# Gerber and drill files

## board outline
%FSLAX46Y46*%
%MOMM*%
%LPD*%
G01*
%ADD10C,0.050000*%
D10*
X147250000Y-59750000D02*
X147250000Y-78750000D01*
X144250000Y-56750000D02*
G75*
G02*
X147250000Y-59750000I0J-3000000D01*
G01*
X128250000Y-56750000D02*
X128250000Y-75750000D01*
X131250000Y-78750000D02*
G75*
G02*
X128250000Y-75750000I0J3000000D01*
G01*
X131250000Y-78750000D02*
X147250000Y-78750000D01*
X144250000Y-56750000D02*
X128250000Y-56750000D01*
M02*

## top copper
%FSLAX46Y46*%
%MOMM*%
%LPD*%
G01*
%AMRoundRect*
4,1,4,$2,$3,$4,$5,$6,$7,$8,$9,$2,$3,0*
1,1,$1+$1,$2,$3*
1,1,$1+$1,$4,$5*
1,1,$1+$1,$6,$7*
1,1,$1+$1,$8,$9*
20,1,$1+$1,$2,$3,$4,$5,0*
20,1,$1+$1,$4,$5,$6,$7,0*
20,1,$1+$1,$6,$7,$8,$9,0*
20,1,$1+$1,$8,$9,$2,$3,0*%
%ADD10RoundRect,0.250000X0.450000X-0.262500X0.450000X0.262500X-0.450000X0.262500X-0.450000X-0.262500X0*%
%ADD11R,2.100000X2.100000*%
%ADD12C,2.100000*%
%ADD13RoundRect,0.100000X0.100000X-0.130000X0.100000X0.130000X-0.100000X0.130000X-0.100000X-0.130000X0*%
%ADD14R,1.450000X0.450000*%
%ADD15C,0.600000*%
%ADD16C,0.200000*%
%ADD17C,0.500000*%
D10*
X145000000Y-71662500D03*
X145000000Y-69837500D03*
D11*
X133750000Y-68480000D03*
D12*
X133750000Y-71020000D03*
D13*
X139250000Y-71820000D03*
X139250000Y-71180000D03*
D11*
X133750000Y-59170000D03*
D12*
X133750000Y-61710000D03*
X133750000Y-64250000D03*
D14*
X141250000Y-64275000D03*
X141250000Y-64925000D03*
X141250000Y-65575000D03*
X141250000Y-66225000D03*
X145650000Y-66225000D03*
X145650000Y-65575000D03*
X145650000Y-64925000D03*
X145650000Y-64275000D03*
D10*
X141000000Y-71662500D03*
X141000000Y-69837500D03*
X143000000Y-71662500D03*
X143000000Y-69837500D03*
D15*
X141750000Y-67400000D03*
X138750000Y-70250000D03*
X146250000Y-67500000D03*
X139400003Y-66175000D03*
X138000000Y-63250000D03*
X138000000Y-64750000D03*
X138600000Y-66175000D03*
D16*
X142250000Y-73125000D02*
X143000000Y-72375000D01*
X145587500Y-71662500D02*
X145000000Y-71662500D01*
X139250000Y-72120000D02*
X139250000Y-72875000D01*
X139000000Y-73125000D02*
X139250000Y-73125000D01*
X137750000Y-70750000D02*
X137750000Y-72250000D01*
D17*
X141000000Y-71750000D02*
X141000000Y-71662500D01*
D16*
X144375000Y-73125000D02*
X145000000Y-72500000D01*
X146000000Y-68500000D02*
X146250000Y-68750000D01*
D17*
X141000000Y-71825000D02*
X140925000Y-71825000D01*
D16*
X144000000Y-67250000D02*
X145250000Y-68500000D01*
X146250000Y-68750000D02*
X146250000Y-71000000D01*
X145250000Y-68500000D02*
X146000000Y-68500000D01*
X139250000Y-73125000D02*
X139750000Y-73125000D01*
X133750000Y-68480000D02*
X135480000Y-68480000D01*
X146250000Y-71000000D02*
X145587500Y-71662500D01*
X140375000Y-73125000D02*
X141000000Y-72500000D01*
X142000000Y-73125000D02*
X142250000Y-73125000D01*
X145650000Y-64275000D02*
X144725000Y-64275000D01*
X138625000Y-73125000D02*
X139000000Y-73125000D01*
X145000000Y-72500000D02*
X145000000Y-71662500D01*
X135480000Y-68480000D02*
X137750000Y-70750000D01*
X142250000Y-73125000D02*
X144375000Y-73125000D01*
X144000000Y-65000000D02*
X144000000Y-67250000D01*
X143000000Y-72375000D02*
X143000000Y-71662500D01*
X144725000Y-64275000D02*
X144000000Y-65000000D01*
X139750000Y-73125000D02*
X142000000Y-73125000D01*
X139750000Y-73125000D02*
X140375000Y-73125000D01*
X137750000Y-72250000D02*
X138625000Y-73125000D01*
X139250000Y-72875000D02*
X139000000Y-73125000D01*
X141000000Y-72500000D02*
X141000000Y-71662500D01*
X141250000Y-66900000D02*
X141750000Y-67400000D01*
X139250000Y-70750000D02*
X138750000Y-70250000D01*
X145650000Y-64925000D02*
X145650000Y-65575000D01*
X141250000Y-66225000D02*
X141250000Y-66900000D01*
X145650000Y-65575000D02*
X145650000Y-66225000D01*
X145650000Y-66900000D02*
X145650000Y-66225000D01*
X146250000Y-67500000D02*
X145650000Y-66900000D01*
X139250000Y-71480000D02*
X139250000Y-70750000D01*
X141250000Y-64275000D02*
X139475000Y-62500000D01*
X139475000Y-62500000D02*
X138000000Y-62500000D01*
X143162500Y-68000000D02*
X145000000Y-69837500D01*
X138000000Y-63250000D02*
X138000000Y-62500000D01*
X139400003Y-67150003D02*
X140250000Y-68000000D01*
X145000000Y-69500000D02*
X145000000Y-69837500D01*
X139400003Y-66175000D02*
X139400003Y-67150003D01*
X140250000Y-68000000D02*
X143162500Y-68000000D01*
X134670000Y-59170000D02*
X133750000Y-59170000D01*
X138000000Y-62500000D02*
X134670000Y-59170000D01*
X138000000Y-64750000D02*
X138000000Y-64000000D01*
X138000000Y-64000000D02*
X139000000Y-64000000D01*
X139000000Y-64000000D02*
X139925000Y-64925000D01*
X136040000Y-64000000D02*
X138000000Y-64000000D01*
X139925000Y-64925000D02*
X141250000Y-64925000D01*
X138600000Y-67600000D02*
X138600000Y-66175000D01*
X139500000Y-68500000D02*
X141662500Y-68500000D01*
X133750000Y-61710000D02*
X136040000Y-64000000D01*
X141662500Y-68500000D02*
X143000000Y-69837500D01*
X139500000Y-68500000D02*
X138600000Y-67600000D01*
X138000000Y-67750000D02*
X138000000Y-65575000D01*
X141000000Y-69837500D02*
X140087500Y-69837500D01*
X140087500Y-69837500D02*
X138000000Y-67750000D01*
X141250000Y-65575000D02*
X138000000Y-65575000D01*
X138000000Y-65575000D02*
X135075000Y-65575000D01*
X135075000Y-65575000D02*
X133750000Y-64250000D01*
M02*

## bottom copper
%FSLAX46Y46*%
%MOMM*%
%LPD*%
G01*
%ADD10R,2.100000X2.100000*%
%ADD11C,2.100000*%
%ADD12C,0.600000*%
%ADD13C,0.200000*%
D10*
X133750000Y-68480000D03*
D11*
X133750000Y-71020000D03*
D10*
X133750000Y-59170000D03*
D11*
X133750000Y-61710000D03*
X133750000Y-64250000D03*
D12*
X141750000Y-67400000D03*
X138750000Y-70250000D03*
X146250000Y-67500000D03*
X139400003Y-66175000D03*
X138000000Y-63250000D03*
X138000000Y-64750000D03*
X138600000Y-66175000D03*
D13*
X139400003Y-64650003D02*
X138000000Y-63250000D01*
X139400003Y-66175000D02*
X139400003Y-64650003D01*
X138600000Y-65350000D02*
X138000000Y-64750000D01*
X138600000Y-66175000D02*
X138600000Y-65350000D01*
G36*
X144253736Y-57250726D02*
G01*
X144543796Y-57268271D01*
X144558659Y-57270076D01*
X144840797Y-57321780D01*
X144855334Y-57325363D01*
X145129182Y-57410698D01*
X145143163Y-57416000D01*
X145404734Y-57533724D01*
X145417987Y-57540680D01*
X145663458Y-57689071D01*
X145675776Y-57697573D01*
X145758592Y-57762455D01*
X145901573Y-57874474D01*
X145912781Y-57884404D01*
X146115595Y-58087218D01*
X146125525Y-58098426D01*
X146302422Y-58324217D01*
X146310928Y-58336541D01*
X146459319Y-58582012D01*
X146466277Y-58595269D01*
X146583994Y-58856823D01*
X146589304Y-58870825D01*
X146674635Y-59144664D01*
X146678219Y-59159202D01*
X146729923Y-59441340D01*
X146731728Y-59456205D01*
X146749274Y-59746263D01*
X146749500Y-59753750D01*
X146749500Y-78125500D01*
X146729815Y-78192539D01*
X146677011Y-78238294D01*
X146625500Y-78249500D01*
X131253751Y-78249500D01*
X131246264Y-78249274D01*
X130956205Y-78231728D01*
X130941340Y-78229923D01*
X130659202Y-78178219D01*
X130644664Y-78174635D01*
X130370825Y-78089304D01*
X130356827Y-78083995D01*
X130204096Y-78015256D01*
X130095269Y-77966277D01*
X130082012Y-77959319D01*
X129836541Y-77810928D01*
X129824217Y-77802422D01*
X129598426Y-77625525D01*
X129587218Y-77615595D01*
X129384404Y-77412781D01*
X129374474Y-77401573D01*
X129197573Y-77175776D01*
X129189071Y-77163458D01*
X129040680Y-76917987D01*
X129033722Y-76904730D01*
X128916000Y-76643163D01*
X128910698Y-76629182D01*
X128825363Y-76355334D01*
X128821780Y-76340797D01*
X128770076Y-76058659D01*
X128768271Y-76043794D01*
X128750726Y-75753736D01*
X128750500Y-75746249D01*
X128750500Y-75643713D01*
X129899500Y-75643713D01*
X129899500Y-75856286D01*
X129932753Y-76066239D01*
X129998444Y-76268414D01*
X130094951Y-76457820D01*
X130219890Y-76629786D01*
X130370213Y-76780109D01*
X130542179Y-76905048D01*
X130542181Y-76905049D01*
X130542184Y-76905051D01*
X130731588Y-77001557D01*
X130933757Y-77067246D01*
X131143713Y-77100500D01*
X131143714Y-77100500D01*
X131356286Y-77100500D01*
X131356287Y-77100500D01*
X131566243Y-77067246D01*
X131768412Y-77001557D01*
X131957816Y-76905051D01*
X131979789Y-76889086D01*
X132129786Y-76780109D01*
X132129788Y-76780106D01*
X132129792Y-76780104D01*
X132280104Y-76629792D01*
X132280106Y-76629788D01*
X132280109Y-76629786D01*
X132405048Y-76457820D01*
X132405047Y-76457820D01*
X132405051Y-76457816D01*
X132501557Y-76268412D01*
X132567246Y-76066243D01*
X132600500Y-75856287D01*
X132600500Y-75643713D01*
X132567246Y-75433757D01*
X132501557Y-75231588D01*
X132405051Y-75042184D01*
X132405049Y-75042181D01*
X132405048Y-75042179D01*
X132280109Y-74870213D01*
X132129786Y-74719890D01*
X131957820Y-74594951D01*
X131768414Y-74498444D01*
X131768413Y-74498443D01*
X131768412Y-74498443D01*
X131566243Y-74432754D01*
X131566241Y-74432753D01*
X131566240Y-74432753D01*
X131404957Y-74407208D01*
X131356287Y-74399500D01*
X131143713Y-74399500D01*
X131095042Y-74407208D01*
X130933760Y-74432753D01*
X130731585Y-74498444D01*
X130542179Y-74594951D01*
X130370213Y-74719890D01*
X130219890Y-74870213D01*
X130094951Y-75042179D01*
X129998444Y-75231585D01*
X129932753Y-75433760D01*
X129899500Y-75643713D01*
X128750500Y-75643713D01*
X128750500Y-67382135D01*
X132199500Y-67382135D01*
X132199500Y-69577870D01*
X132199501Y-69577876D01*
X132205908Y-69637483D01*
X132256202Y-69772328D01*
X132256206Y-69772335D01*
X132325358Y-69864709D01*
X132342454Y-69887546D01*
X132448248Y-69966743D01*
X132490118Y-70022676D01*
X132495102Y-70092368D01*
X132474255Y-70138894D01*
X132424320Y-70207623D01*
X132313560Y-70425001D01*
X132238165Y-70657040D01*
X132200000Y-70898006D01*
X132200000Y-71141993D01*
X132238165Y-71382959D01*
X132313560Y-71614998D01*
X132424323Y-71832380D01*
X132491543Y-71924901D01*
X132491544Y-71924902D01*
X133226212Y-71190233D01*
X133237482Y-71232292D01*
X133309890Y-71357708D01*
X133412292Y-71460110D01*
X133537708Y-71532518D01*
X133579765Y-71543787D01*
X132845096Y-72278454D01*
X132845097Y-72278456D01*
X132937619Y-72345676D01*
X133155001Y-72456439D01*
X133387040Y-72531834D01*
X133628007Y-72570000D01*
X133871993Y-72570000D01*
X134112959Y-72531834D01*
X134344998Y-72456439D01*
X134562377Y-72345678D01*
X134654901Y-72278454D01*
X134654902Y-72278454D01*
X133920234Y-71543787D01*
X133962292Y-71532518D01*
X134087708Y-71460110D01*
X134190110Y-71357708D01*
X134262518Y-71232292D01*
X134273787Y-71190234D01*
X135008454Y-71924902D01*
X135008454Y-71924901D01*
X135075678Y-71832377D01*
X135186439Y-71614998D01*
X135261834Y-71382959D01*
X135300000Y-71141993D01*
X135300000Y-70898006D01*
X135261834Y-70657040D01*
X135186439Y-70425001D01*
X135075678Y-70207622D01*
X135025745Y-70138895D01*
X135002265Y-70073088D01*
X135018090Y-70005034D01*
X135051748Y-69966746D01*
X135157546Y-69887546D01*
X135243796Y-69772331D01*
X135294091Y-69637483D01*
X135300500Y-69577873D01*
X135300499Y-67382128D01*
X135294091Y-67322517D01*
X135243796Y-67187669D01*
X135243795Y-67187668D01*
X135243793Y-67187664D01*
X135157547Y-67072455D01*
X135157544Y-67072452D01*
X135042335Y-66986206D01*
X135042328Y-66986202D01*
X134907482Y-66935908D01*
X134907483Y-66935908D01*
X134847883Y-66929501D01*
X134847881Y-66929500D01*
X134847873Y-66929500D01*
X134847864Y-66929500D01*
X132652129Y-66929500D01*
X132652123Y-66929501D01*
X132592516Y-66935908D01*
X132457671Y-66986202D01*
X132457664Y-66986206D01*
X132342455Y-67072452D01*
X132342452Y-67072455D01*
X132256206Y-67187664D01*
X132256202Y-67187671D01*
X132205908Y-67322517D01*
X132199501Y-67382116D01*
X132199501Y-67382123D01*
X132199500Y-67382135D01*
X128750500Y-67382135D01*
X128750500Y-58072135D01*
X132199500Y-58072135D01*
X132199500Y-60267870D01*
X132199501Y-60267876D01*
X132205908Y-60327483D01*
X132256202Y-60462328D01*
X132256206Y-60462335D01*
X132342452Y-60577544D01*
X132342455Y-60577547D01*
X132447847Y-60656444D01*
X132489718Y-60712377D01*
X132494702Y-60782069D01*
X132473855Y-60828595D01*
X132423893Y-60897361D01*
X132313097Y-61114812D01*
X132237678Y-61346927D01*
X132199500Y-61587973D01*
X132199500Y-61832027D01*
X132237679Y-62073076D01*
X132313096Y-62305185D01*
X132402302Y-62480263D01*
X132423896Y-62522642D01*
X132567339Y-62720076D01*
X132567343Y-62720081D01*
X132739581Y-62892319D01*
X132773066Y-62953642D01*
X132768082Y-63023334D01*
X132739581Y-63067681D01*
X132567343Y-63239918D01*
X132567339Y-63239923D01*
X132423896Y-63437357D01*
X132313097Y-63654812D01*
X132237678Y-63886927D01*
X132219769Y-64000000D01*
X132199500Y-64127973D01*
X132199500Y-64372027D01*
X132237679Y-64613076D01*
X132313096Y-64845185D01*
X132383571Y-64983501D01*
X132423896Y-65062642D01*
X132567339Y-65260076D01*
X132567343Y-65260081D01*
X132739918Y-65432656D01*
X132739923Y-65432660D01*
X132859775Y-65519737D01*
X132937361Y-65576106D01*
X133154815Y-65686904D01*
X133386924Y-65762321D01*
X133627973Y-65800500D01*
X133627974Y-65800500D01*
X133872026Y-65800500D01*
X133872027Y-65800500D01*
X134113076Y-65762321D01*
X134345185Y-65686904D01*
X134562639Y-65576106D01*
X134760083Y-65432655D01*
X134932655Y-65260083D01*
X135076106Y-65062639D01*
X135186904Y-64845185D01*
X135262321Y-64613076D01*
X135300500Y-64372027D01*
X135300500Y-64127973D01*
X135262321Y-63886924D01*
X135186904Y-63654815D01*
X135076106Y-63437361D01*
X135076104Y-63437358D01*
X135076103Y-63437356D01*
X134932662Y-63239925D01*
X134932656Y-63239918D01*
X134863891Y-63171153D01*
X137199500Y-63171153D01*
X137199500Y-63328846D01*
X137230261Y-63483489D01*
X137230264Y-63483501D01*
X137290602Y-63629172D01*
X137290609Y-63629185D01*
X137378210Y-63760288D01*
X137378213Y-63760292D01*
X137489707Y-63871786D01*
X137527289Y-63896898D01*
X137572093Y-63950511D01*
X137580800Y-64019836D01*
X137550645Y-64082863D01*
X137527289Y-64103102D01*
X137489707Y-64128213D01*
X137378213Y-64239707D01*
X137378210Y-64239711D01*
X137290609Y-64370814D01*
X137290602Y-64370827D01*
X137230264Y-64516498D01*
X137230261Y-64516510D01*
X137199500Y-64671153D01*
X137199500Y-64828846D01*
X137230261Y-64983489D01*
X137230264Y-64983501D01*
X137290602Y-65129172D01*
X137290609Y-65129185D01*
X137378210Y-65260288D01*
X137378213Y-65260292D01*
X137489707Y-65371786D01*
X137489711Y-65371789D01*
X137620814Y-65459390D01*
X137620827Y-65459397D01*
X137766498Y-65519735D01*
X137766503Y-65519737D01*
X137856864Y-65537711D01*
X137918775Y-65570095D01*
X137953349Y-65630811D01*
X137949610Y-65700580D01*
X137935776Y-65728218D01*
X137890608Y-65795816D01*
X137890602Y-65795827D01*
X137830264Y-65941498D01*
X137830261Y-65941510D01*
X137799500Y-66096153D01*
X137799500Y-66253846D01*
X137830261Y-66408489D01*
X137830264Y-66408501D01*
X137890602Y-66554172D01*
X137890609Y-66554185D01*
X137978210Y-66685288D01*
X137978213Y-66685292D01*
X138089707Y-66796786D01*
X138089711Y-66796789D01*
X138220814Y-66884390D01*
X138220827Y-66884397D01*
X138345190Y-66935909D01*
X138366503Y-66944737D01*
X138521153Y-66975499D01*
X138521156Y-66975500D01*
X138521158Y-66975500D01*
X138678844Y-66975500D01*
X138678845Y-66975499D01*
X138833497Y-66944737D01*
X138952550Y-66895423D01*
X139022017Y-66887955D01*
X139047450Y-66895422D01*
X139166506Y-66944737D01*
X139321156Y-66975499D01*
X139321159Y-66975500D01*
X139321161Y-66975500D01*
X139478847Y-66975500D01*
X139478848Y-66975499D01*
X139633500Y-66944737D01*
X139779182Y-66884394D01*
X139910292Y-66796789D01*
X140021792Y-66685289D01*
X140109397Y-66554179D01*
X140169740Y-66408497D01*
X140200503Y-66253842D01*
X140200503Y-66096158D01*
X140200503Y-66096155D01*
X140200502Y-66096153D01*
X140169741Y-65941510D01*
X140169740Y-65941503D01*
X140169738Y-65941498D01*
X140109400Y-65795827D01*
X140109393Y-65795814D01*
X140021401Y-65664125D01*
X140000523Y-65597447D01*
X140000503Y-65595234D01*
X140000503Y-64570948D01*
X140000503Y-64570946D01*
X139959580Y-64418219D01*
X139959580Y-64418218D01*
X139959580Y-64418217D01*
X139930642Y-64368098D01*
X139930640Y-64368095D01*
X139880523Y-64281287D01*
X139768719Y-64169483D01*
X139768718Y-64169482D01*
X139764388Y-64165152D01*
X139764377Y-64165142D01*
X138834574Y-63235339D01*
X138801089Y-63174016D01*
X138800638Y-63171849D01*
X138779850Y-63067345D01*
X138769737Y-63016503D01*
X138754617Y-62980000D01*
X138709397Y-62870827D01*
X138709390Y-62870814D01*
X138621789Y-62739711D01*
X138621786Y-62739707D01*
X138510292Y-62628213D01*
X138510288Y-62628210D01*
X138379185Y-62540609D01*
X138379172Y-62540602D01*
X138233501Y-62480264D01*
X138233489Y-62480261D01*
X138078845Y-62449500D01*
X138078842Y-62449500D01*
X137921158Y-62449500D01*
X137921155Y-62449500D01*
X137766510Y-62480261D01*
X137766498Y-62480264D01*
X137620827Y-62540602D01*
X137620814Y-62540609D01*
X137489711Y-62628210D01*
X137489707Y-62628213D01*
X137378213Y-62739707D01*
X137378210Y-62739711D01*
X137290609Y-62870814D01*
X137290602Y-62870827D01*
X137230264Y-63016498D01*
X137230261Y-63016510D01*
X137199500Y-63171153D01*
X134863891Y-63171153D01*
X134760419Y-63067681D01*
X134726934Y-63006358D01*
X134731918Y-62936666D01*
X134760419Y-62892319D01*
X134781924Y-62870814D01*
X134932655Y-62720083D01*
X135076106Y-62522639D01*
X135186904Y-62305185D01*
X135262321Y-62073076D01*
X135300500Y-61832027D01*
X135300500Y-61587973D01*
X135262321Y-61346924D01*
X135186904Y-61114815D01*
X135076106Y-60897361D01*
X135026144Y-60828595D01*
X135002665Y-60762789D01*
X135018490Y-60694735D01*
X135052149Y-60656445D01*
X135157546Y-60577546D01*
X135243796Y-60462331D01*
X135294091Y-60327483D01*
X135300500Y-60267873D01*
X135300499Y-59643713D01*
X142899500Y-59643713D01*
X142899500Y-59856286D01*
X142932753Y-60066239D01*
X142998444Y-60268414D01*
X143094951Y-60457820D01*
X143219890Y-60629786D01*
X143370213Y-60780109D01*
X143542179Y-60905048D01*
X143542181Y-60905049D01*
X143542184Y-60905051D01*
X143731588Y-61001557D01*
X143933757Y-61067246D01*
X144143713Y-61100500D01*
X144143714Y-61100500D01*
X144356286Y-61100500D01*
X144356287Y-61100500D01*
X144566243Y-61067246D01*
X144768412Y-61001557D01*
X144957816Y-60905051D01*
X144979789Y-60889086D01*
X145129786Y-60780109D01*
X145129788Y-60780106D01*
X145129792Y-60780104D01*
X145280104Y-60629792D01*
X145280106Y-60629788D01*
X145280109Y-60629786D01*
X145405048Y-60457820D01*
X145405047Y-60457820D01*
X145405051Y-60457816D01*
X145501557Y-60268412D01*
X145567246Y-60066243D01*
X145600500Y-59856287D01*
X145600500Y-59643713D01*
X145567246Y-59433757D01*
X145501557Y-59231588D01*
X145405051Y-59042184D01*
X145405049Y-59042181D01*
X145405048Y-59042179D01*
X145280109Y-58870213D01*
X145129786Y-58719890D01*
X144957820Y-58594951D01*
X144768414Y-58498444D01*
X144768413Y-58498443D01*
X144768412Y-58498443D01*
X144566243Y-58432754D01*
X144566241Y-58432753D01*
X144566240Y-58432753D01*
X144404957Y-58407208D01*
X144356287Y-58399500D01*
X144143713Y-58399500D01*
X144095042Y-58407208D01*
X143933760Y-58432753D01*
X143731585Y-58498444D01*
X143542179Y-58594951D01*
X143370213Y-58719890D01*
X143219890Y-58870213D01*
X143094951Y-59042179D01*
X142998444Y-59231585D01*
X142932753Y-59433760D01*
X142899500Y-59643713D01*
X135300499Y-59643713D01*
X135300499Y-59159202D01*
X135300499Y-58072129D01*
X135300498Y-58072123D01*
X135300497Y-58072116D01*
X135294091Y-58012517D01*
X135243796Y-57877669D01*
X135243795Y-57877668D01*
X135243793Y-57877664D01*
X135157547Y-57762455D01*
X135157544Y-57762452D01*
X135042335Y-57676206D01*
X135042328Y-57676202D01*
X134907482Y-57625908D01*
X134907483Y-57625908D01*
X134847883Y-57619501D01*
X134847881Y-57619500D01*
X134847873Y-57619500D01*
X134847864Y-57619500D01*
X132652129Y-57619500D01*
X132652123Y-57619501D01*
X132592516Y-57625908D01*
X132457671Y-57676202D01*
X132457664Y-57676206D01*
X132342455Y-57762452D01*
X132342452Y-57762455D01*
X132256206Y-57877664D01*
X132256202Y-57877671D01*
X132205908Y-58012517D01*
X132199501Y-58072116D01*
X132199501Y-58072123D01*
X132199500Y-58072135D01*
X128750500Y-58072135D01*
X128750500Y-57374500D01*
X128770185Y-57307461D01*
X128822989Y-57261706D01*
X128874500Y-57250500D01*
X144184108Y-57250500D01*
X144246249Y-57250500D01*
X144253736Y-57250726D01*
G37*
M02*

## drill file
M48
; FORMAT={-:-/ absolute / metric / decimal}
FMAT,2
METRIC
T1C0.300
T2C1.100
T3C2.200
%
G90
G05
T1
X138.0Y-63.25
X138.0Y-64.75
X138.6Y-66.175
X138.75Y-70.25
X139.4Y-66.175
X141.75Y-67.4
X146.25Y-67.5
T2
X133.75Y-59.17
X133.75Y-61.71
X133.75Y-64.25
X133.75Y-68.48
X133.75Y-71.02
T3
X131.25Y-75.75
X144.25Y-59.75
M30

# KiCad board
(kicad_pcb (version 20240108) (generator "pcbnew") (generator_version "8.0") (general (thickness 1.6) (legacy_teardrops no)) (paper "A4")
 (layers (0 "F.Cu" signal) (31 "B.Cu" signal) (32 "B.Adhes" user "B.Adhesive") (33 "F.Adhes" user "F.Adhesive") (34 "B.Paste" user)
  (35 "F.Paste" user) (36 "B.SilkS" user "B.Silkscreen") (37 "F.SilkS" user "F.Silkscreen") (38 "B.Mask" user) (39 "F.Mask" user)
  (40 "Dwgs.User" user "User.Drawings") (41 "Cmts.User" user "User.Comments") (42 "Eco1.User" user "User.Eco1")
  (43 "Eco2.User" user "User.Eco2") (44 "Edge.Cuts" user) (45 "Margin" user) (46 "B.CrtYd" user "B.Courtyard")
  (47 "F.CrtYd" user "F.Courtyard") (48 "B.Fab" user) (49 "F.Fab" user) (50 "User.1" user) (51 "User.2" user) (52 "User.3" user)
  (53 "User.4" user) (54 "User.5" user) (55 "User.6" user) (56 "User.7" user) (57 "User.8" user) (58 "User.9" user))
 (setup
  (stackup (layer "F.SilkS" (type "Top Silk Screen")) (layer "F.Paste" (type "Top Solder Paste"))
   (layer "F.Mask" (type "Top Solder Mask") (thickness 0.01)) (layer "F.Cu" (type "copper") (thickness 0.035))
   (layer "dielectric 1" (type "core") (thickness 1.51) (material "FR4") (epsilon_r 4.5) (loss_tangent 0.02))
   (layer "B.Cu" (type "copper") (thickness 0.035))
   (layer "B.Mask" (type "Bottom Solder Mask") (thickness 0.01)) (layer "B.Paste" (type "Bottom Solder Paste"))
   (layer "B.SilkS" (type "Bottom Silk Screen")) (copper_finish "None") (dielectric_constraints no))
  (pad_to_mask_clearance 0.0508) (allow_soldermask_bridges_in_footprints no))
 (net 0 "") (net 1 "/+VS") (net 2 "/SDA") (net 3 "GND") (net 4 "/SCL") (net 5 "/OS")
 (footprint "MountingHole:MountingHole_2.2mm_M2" (layer "F.Cu") (at 144.25 59.75)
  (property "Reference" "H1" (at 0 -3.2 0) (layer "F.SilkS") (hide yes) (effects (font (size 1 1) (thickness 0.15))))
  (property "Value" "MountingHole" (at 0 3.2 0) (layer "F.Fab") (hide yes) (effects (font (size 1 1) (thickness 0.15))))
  (pad "" np_thru_hole circle (at 0 0) (size 2.2 2.2) (drill 2.2) (layers "*.Cu" "*.Mask")))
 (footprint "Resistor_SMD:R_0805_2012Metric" (layer "F.Cu") (at 145 70.75 90)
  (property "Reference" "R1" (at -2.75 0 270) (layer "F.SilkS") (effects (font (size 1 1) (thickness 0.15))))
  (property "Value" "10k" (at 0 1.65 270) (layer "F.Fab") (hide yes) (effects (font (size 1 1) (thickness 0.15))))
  (pad "1" smd roundrect (at -0.9125 0 90) (size 1.025 1.4) (layers "F.Cu" "F.Paste" "F.Mask") (roundrect_rratio 0.243902) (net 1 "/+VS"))
  (pad "2" smd roundrect (at 0.9125 0 90) (size 1.025 1.4) (layers "F.Cu" "F.Paste" "F.Mask") (roundrect_rratio 0.243902) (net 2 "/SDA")))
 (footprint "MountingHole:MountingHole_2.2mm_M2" (layer "F.Cu") (at 131.25 75.75)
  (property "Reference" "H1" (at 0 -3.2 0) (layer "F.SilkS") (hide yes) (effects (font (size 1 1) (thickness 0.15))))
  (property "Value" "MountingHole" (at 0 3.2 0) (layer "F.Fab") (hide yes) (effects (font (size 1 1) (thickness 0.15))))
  (pad "" np_thru_hole circle (at 0 0) (size 2.2 2.2) (drill 2.2) (layers "F&B.Cu" "*.Mask")))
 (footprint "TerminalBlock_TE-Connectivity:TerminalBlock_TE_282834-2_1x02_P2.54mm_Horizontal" (layer "F.Cu") (at 133.75 68.48 -90)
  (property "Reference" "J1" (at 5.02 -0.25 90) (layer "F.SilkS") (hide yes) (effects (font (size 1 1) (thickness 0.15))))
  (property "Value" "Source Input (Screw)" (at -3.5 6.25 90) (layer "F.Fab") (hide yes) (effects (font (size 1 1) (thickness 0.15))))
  (pad "1" thru_hole rect (at 0 0 270) (size 2.1 2.1) (drill 1.1) (layers "*.Cu" "*.Mask") (remove_unused_layers no) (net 1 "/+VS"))
  (pad "2" thru_hole circle (at 2.54 0 270) (size 2.1 2.1) (drill 1.1) (layers "*.Cu" "*.Mask") (remove_unused_layers no) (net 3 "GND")))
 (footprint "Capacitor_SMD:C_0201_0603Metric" (layer "F.Cu") (at 139.25 71.5 90)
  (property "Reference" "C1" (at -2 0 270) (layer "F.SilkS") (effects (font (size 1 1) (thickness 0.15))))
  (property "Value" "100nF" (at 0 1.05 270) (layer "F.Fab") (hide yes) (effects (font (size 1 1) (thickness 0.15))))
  (pad "" smd roundrect (at -0.345 0 90) (size 0.318 0.36) (layers "F.Paste") (roundrect_rratio 0.25))
  (pad "" smd roundrect (at 0.345 0 90) (size 0.318 0.36) (layers "F.Paste") (roundrect_rratio 0.25))
  (pad "1" smd roundrect (at -0.32 0 90) (size 0.46 0.4) (layers "F.Cu" "F.Mask") (roundrect_rratio 0.25) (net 1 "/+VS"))
  (pad "2" smd roundrect (at 0.32 0 90) (size 0.46 0.4) (layers "F.Cu" "F.Mask") (roundrect_rratio 0.25) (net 3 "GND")))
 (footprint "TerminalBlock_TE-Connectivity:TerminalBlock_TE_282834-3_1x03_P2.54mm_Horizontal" (layer "F.Cu") (at 133.75 59.17 -90)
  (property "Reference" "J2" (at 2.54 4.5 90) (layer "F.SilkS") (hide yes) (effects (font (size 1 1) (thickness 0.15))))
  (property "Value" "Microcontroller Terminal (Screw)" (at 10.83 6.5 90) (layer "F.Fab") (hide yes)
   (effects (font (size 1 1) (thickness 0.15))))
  (pad "1" thru_hole rect (at 0 0 270) (size 2.1 2.1) (drill 1.1) (layers "*.Cu" "*.Mask") (remove_unused_layers no) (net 2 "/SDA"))
  (pad "2" thru_hole circle (at 2.54 0 270) (size 2.1 2.1) (drill 1.1) (layers "*.Cu" "*.Mask") (remove_unused_layers no) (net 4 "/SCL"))
  (pad "3" thru_hole circle (at 5.08 0 270) (size 2.1 2.1) (drill 1.1) (layers "*.Cu" "*.Mask") (remove_unused_layers no) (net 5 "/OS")))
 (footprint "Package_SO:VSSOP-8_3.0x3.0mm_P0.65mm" (layer "F.Cu") (at 143.45 65.25)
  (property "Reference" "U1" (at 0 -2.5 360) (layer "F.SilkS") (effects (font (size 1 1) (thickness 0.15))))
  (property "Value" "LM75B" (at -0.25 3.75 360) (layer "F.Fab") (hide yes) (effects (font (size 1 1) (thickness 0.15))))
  (pad "1" smd rect (at -2.2 -0.975 270) (size 0.45 1.45) (layers "F.Cu" "F.Paste" "F.Mask") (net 2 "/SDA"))
  (pad "2" smd rect (at -2.2 -0.325 270) (size 0.45 1.45) (layers "F.Cu" "F.Paste" "F.Mask") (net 4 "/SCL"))
  (pad "3" smd rect (at -2.2 0.325 270) (size 0.45 1.45) (layers "F.Cu" "F.Paste" "F.Mask") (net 5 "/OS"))
  (pad "4" smd rect (at -2.2 0.975 270) (size 0.45 1.45) (layers "F.Cu" "F.Paste" "F.Mask") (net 3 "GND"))
  (pad "5" smd rect (at 2.2 0.975 270) (size 0.45 1.45) (layers "F.Cu" "F.Paste" "F.Mask") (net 3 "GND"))
  (pad "6" smd rect (at 2.2 0.325 270) (size 0.45 1.45) (layers "F.Cu" "F.Paste" "F.Mask") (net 3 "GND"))
  (pad "7" smd rect (at 2.2 -0.325 270) (size 0.45 1.45) (layers "F.Cu" "F.Paste" "F.Mask") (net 3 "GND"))
  (pad "8" smd rect (at 2.2 -0.975 270) (size 0.45 1.45) (layers "F.Cu" "F.Paste" "F.Mask") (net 1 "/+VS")))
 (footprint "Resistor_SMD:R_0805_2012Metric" (layer "F.Cu") (at 141 70.75 90)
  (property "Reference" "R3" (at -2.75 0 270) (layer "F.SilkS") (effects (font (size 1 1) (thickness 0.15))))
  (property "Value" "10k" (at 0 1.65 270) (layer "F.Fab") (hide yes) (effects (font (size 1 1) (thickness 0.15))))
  (pad "1" smd roundrect (at -0.9125 0 90) (size 1.025 1.4) (layers "F.Cu" "F.Paste" "F.Mask") (roundrect_rratio 0.243902) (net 1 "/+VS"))
  (pad "2" smd roundrect (at 0.9125 0 90) (size 1.025 1.4) (layers "F.Cu" "F.Paste" "F.Mask") (roundrect_rratio 0.243902) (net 5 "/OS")))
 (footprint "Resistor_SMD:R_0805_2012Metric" (layer "F.Cu") (at 143 70.75 90)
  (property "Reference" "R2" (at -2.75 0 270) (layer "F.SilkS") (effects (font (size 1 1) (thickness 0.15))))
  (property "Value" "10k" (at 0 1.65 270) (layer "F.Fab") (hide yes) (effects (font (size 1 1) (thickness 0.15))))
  (pad "1" smd roundrect (at -0.9125 0 90) (size 1.025 1.4) (layers "F.Cu" "F.Paste" "F.Mask") (roundrect_rratio 0.243902) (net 1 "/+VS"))
  (pad "2" smd roundrect (at 0.9125 0 90) (size 1.025 1.4) (layers "F.Cu" "F.Paste" "F.Mask") (roundrect_rratio 0.243902) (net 4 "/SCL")))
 (gr_line (start 147.25 59.75) (end 147.25 78.75) (stroke (width 0.05) (type default)) (layer "Edge.Cuts"))
 (gr_arc (start 144.25 56.75) (mid 146.37132 57.62868) (end 147.25 59.75) (stroke (width 0.05) (type default)) (layer "Edge.Cuts"))
 (gr_line (start 128.25 56.75) (end 128.25 75.75) (stroke (width 0.05) (type default)) (layer "Edge.Cuts"))
 (gr_arc (start 131.25 78.75) (mid 129.12868 77.87132) (end 128.25 75.75) (stroke (width 0.05) (type default)) (layer "Edge.Cuts"))
 (gr_line (start 131.25 78.75) (end 147.25 78.75) (stroke (width 0.05) (type default)) (layer "Edge.Cuts"))
 (gr_line (start 144.25 56.75) (end 128.25 56.75) (stroke (width 0.05) (type default)) (layer "Edge.Cuts"))
 (segment (start 142.25 73.125) (end 143 72.375) (width 0.2) (layer "F.Cu") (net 1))
 (segment (start 145.5875 71.6625) (end 145 71.6625) (width 0.2) (layer "F.Cu") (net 1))
 (segment (start 139.25 72.12) (end 139.25 72.875) (width 0.2) (layer "F.Cu") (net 1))
 (segment (start 139 73.125) (end 139.25 73.125) (width 0.2) (layer "F.Cu") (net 1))
 (segment (start 137.75 70.75) (end 137.75 72.25) (width 0.2) (layer "F.Cu") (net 1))
 (segment (start 141 71.75) (end 141 71.6625) (width 0.5) (layer "F.Cu") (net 1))
 (segment (start 144.375 73.125) (end 145 72.5) (width 0.2) (layer "F.Cu") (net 1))
 (segment (start 146 68.5) (end 146.25 68.75) (width 0.2) (layer "F.Cu") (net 1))
 (segment (start 141 71.825) (end 140.925 71.825) (width 0.5) (layer "F.Cu") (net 1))
 (segment (start 144 67.25) (end 145.25 68.5) (width 0.2) (layer "F.Cu") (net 1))
 (segment (start 146.25 68.75) (end 146.25 71) (width 0.2) (layer "F.Cu") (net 1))
 (segment (start 145.25 68.5) (end 146 68.5) (width 0.2) (layer "F.Cu") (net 1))
 (segment (start 139.25 73.125) (end 139.75 73.125) (width 0.2) (layer "F.Cu") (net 1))
 (segment (start 133.75 68.48) (end 135.48 68.48) (width 0.2) (layer "F.Cu") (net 1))
 (segment (start 146.25 71) (end 145.5875 71.6625) (width 0.2) (layer "F.Cu") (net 1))
 (segment (start 140.375 73.125) (end 141 72.5) (width 0.2) (layer "F.Cu") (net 1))
 (segment (start 142 73.125) (end 142.25 73.125) (width 0.2) (layer "F.Cu") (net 1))
 (segment (start 145.65 64.275) (end 144.725 64.275) (width 0.2) (layer "F.Cu") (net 1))
 (segment (start 138.625 73.125) (end 139 73.125) (width 0.2) (layer "F.Cu") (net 1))
 (segment (start 145 72.5) (end 145 71.6625) (width 0.2) (layer "F.Cu") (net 1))
 (segment (start 135.48 68.48) (end 137.75 70.75) (width 0.2) (layer "F.Cu") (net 1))
 (segment (start 142.25 73.125) (end 144.375 73.125) (width 0.2) (layer "F.Cu") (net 1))
 (segment (start 144 65) (end 144 67.25) (width 0.2) (layer "F.Cu") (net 1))
 (segment (start 143 72.375) (end 143 71.6625) (width 0.2) (layer "F.Cu") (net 1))
 (segment (start 144.725 64.275) (end 144 65) (width 0.2) (layer "F.Cu") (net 1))
 (segment (start 139.75 73.125) (end 142 73.125) (width 0.2) (layer "F.Cu") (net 1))
 (segment (start 139.75 73.125) (end 140.375 73.125) (width 0.2) (layer "F.Cu") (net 1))
 (segment (start 137.75 72.25) (end 138.625 73.125) (width 0.2) (layer "F.Cu") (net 1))
 (segment (start 139.25 72.875) (end 139 73.125) (width 0.2) (layer "F.Cu") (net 1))
 (segment (start 141 72.5) (end 141 71.6625) (width 0.2) (layer "F.Cu") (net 1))
 (segment (start 141.25 66.9) (end 141.75 67.4) (width 0.2) (layer "F.Cu") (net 3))
 (segment (start 139.25 70.75) (end 138.75 70.25) (width 0.2) (layer "F.Cu") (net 3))
 (segment (start 145.65 64.925) (end 145.65 65.575) (width 0.2) (layer "F.Cu") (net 3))
 (segment (start 141.25 66.225) (end 141.25 66.9) (width 0.2) (layer "F.Cu") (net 3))
 (segment (start 145.65 65.575) (end 145.65 66.225) (width 0.2) (layer "F.Cu") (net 3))
 (segment (start 145.65 66.9) (end 145.65 66.225) (width 0.2) (layer "F.Cu") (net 3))
 (segment (start 146.25 67.5) (end 145.65 66.9) (width 0.2) (layer "F.Cu") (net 3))
 (segment (start 139.25 71.48) (end 139.25 70.75) (width 0.2) (layer "F.Cu") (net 3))
 (via (at 141.75 67.4) (size 0.6) (drill 0.3) (layers "F.Cu" "B.Cu") (free yes) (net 3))
 (via (at 138.75 70.25) (size 0.6) (drill 0.3) (layers "F.Cu" "B.Cu") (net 3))
 (via (at 146.25 67.5) (size 0.6) (drill 0.3) (layers "F.Cu" "B.Cu") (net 3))
 (segment (start 141.25 64.275) (end 139.475 62.5) (width 0.2) (layer "F.Cu") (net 2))
 (segment (start 139.475 62.5) (end 138 62.5) (width 0.2) (layer "F.Cu") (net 2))
 (segment (start 143.1625 68) (end 145 69.8375) (width 0.2) (layer "F.Cu") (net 2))
 (segment (start 138 63.25) (end 138 62.5) (width 0.2) (layer "F.Cu") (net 2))
 (segment (start 139.400003 67.150003) (end 140.25 68) (width 0.2) (layer "F.Cu") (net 2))
 (segment (start 145 69.5) (end 145 69.8375) (width 0.2) (layer "F.Cu") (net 2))
 (segment (start 139.400003 66.175) (end 139.400003 67.150003) (width 0.2) (layer "F.Cu") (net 2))
 (segment (start 140.25 68) (end 143.1625 68) (width 0.2) (layer "F.Cu") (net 2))
 (segment (start 134.67 59.17) (end 133.75 59.17) (width 0.2) (layer "F.Cu") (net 2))
 (segment (start 138 62.5) (end 134.67 59.17) (width 0.2) (layer "F.Cu") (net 2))
 (via (at 139.400003 66.175) (size 0.6) (drill 0.3) (layers "F.Cu" "B.Cu") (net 2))
 (via (at 138 63.25) (size 0.6) (drill 0.3) (layers "F.Cu" "B.Cu") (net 2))
 (segment (start 139.400003 64.650003) (end 138 63.25) (width 0.2) (layer "B.Cu") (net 2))
 (segment (start 139.400003 66.175) (end 139.400003 64.650003) (width 0.2) (layer "B.Cu") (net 2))
 (segment (start 138 64.75) (end 138 64) (width 0.2) (layer "F.Cu") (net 4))
 (segment (start 138 64) (end 139 64) (width 0.2) (layer "F.Cu") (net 4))
 (segment (start 139 64) (end 139.925 64.925) (width 0.2) (layer "F.Cu") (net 4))
 (segment (start 136.04 64) (end 138 64) (width 0.2) (layer "F.Cu") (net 4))
 (segment (start 139.925 64.925) (end 141.25 64.925) (width 0.2) (layer "F.Cu") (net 4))
 (segment (start 138.6 67.6) (end 138.6 66.175) (width 0.2) (layer "F.Cu") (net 4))
 (segment (start 139.5 68.5) (end 141.6625 68.5) (width 0.2) (layer "F.Cu") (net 4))
 (segment (start 133.75 61.71) (end 136.04 64) (width 0.2) (layer "F.Cu") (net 4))
 (segment (start 141.6625 68.5) (end 143 69.8375) (width 0.2) (layer "F.Cu") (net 4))
 (segment (start 139.5 68.5) (end 138.6 67.6) (width 0.2) (layer "F.Cu") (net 4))
 (via (at 138 64.75) (size 0.6) (drill 0.3) (layers "F.Cu" "B.Cu") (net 4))
 (via (at 138.6 66.175) (size 0.6) (drill 0.3) (layers "F.Cu" "B.Cu") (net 4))
 (segment (start 138.6 65.35) (end 138 64.75) (width 0.2) (layer "B.Cu") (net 4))
 (segment (start 138.6 66.175) (end 138.6 65.35) (width 0.2) (layer "B.Cu") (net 4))
 (segment (start 138 67.75) (end 138 65.575) (width 0.2) (layer "F.Cu") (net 5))
 (segment (start 141 69.8375) (end 140.0875 69.8375) (width 0.2) (layer "F.Cu") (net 5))
 (segment (start 140.0875 69.8375) (end 138 67.75) (width 0.2) (layer "F.Cu") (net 5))
 (segment (start 141.25 65.575) (end 138 65.575) (width 0.2) (layer "F.Cu") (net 5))
 (segment (start 138 65.575) (end 135.075 65.575) (width 0.2) (layer "F.Cu") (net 5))
 (segment (start 135.075 65.575) (end 133.75 64.25) (width 0.2) (layer "F.Cu") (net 5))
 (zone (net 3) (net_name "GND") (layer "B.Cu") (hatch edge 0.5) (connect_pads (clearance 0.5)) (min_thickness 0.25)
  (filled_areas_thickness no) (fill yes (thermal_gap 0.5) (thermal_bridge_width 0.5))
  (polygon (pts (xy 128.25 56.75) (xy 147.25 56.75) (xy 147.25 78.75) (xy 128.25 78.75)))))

